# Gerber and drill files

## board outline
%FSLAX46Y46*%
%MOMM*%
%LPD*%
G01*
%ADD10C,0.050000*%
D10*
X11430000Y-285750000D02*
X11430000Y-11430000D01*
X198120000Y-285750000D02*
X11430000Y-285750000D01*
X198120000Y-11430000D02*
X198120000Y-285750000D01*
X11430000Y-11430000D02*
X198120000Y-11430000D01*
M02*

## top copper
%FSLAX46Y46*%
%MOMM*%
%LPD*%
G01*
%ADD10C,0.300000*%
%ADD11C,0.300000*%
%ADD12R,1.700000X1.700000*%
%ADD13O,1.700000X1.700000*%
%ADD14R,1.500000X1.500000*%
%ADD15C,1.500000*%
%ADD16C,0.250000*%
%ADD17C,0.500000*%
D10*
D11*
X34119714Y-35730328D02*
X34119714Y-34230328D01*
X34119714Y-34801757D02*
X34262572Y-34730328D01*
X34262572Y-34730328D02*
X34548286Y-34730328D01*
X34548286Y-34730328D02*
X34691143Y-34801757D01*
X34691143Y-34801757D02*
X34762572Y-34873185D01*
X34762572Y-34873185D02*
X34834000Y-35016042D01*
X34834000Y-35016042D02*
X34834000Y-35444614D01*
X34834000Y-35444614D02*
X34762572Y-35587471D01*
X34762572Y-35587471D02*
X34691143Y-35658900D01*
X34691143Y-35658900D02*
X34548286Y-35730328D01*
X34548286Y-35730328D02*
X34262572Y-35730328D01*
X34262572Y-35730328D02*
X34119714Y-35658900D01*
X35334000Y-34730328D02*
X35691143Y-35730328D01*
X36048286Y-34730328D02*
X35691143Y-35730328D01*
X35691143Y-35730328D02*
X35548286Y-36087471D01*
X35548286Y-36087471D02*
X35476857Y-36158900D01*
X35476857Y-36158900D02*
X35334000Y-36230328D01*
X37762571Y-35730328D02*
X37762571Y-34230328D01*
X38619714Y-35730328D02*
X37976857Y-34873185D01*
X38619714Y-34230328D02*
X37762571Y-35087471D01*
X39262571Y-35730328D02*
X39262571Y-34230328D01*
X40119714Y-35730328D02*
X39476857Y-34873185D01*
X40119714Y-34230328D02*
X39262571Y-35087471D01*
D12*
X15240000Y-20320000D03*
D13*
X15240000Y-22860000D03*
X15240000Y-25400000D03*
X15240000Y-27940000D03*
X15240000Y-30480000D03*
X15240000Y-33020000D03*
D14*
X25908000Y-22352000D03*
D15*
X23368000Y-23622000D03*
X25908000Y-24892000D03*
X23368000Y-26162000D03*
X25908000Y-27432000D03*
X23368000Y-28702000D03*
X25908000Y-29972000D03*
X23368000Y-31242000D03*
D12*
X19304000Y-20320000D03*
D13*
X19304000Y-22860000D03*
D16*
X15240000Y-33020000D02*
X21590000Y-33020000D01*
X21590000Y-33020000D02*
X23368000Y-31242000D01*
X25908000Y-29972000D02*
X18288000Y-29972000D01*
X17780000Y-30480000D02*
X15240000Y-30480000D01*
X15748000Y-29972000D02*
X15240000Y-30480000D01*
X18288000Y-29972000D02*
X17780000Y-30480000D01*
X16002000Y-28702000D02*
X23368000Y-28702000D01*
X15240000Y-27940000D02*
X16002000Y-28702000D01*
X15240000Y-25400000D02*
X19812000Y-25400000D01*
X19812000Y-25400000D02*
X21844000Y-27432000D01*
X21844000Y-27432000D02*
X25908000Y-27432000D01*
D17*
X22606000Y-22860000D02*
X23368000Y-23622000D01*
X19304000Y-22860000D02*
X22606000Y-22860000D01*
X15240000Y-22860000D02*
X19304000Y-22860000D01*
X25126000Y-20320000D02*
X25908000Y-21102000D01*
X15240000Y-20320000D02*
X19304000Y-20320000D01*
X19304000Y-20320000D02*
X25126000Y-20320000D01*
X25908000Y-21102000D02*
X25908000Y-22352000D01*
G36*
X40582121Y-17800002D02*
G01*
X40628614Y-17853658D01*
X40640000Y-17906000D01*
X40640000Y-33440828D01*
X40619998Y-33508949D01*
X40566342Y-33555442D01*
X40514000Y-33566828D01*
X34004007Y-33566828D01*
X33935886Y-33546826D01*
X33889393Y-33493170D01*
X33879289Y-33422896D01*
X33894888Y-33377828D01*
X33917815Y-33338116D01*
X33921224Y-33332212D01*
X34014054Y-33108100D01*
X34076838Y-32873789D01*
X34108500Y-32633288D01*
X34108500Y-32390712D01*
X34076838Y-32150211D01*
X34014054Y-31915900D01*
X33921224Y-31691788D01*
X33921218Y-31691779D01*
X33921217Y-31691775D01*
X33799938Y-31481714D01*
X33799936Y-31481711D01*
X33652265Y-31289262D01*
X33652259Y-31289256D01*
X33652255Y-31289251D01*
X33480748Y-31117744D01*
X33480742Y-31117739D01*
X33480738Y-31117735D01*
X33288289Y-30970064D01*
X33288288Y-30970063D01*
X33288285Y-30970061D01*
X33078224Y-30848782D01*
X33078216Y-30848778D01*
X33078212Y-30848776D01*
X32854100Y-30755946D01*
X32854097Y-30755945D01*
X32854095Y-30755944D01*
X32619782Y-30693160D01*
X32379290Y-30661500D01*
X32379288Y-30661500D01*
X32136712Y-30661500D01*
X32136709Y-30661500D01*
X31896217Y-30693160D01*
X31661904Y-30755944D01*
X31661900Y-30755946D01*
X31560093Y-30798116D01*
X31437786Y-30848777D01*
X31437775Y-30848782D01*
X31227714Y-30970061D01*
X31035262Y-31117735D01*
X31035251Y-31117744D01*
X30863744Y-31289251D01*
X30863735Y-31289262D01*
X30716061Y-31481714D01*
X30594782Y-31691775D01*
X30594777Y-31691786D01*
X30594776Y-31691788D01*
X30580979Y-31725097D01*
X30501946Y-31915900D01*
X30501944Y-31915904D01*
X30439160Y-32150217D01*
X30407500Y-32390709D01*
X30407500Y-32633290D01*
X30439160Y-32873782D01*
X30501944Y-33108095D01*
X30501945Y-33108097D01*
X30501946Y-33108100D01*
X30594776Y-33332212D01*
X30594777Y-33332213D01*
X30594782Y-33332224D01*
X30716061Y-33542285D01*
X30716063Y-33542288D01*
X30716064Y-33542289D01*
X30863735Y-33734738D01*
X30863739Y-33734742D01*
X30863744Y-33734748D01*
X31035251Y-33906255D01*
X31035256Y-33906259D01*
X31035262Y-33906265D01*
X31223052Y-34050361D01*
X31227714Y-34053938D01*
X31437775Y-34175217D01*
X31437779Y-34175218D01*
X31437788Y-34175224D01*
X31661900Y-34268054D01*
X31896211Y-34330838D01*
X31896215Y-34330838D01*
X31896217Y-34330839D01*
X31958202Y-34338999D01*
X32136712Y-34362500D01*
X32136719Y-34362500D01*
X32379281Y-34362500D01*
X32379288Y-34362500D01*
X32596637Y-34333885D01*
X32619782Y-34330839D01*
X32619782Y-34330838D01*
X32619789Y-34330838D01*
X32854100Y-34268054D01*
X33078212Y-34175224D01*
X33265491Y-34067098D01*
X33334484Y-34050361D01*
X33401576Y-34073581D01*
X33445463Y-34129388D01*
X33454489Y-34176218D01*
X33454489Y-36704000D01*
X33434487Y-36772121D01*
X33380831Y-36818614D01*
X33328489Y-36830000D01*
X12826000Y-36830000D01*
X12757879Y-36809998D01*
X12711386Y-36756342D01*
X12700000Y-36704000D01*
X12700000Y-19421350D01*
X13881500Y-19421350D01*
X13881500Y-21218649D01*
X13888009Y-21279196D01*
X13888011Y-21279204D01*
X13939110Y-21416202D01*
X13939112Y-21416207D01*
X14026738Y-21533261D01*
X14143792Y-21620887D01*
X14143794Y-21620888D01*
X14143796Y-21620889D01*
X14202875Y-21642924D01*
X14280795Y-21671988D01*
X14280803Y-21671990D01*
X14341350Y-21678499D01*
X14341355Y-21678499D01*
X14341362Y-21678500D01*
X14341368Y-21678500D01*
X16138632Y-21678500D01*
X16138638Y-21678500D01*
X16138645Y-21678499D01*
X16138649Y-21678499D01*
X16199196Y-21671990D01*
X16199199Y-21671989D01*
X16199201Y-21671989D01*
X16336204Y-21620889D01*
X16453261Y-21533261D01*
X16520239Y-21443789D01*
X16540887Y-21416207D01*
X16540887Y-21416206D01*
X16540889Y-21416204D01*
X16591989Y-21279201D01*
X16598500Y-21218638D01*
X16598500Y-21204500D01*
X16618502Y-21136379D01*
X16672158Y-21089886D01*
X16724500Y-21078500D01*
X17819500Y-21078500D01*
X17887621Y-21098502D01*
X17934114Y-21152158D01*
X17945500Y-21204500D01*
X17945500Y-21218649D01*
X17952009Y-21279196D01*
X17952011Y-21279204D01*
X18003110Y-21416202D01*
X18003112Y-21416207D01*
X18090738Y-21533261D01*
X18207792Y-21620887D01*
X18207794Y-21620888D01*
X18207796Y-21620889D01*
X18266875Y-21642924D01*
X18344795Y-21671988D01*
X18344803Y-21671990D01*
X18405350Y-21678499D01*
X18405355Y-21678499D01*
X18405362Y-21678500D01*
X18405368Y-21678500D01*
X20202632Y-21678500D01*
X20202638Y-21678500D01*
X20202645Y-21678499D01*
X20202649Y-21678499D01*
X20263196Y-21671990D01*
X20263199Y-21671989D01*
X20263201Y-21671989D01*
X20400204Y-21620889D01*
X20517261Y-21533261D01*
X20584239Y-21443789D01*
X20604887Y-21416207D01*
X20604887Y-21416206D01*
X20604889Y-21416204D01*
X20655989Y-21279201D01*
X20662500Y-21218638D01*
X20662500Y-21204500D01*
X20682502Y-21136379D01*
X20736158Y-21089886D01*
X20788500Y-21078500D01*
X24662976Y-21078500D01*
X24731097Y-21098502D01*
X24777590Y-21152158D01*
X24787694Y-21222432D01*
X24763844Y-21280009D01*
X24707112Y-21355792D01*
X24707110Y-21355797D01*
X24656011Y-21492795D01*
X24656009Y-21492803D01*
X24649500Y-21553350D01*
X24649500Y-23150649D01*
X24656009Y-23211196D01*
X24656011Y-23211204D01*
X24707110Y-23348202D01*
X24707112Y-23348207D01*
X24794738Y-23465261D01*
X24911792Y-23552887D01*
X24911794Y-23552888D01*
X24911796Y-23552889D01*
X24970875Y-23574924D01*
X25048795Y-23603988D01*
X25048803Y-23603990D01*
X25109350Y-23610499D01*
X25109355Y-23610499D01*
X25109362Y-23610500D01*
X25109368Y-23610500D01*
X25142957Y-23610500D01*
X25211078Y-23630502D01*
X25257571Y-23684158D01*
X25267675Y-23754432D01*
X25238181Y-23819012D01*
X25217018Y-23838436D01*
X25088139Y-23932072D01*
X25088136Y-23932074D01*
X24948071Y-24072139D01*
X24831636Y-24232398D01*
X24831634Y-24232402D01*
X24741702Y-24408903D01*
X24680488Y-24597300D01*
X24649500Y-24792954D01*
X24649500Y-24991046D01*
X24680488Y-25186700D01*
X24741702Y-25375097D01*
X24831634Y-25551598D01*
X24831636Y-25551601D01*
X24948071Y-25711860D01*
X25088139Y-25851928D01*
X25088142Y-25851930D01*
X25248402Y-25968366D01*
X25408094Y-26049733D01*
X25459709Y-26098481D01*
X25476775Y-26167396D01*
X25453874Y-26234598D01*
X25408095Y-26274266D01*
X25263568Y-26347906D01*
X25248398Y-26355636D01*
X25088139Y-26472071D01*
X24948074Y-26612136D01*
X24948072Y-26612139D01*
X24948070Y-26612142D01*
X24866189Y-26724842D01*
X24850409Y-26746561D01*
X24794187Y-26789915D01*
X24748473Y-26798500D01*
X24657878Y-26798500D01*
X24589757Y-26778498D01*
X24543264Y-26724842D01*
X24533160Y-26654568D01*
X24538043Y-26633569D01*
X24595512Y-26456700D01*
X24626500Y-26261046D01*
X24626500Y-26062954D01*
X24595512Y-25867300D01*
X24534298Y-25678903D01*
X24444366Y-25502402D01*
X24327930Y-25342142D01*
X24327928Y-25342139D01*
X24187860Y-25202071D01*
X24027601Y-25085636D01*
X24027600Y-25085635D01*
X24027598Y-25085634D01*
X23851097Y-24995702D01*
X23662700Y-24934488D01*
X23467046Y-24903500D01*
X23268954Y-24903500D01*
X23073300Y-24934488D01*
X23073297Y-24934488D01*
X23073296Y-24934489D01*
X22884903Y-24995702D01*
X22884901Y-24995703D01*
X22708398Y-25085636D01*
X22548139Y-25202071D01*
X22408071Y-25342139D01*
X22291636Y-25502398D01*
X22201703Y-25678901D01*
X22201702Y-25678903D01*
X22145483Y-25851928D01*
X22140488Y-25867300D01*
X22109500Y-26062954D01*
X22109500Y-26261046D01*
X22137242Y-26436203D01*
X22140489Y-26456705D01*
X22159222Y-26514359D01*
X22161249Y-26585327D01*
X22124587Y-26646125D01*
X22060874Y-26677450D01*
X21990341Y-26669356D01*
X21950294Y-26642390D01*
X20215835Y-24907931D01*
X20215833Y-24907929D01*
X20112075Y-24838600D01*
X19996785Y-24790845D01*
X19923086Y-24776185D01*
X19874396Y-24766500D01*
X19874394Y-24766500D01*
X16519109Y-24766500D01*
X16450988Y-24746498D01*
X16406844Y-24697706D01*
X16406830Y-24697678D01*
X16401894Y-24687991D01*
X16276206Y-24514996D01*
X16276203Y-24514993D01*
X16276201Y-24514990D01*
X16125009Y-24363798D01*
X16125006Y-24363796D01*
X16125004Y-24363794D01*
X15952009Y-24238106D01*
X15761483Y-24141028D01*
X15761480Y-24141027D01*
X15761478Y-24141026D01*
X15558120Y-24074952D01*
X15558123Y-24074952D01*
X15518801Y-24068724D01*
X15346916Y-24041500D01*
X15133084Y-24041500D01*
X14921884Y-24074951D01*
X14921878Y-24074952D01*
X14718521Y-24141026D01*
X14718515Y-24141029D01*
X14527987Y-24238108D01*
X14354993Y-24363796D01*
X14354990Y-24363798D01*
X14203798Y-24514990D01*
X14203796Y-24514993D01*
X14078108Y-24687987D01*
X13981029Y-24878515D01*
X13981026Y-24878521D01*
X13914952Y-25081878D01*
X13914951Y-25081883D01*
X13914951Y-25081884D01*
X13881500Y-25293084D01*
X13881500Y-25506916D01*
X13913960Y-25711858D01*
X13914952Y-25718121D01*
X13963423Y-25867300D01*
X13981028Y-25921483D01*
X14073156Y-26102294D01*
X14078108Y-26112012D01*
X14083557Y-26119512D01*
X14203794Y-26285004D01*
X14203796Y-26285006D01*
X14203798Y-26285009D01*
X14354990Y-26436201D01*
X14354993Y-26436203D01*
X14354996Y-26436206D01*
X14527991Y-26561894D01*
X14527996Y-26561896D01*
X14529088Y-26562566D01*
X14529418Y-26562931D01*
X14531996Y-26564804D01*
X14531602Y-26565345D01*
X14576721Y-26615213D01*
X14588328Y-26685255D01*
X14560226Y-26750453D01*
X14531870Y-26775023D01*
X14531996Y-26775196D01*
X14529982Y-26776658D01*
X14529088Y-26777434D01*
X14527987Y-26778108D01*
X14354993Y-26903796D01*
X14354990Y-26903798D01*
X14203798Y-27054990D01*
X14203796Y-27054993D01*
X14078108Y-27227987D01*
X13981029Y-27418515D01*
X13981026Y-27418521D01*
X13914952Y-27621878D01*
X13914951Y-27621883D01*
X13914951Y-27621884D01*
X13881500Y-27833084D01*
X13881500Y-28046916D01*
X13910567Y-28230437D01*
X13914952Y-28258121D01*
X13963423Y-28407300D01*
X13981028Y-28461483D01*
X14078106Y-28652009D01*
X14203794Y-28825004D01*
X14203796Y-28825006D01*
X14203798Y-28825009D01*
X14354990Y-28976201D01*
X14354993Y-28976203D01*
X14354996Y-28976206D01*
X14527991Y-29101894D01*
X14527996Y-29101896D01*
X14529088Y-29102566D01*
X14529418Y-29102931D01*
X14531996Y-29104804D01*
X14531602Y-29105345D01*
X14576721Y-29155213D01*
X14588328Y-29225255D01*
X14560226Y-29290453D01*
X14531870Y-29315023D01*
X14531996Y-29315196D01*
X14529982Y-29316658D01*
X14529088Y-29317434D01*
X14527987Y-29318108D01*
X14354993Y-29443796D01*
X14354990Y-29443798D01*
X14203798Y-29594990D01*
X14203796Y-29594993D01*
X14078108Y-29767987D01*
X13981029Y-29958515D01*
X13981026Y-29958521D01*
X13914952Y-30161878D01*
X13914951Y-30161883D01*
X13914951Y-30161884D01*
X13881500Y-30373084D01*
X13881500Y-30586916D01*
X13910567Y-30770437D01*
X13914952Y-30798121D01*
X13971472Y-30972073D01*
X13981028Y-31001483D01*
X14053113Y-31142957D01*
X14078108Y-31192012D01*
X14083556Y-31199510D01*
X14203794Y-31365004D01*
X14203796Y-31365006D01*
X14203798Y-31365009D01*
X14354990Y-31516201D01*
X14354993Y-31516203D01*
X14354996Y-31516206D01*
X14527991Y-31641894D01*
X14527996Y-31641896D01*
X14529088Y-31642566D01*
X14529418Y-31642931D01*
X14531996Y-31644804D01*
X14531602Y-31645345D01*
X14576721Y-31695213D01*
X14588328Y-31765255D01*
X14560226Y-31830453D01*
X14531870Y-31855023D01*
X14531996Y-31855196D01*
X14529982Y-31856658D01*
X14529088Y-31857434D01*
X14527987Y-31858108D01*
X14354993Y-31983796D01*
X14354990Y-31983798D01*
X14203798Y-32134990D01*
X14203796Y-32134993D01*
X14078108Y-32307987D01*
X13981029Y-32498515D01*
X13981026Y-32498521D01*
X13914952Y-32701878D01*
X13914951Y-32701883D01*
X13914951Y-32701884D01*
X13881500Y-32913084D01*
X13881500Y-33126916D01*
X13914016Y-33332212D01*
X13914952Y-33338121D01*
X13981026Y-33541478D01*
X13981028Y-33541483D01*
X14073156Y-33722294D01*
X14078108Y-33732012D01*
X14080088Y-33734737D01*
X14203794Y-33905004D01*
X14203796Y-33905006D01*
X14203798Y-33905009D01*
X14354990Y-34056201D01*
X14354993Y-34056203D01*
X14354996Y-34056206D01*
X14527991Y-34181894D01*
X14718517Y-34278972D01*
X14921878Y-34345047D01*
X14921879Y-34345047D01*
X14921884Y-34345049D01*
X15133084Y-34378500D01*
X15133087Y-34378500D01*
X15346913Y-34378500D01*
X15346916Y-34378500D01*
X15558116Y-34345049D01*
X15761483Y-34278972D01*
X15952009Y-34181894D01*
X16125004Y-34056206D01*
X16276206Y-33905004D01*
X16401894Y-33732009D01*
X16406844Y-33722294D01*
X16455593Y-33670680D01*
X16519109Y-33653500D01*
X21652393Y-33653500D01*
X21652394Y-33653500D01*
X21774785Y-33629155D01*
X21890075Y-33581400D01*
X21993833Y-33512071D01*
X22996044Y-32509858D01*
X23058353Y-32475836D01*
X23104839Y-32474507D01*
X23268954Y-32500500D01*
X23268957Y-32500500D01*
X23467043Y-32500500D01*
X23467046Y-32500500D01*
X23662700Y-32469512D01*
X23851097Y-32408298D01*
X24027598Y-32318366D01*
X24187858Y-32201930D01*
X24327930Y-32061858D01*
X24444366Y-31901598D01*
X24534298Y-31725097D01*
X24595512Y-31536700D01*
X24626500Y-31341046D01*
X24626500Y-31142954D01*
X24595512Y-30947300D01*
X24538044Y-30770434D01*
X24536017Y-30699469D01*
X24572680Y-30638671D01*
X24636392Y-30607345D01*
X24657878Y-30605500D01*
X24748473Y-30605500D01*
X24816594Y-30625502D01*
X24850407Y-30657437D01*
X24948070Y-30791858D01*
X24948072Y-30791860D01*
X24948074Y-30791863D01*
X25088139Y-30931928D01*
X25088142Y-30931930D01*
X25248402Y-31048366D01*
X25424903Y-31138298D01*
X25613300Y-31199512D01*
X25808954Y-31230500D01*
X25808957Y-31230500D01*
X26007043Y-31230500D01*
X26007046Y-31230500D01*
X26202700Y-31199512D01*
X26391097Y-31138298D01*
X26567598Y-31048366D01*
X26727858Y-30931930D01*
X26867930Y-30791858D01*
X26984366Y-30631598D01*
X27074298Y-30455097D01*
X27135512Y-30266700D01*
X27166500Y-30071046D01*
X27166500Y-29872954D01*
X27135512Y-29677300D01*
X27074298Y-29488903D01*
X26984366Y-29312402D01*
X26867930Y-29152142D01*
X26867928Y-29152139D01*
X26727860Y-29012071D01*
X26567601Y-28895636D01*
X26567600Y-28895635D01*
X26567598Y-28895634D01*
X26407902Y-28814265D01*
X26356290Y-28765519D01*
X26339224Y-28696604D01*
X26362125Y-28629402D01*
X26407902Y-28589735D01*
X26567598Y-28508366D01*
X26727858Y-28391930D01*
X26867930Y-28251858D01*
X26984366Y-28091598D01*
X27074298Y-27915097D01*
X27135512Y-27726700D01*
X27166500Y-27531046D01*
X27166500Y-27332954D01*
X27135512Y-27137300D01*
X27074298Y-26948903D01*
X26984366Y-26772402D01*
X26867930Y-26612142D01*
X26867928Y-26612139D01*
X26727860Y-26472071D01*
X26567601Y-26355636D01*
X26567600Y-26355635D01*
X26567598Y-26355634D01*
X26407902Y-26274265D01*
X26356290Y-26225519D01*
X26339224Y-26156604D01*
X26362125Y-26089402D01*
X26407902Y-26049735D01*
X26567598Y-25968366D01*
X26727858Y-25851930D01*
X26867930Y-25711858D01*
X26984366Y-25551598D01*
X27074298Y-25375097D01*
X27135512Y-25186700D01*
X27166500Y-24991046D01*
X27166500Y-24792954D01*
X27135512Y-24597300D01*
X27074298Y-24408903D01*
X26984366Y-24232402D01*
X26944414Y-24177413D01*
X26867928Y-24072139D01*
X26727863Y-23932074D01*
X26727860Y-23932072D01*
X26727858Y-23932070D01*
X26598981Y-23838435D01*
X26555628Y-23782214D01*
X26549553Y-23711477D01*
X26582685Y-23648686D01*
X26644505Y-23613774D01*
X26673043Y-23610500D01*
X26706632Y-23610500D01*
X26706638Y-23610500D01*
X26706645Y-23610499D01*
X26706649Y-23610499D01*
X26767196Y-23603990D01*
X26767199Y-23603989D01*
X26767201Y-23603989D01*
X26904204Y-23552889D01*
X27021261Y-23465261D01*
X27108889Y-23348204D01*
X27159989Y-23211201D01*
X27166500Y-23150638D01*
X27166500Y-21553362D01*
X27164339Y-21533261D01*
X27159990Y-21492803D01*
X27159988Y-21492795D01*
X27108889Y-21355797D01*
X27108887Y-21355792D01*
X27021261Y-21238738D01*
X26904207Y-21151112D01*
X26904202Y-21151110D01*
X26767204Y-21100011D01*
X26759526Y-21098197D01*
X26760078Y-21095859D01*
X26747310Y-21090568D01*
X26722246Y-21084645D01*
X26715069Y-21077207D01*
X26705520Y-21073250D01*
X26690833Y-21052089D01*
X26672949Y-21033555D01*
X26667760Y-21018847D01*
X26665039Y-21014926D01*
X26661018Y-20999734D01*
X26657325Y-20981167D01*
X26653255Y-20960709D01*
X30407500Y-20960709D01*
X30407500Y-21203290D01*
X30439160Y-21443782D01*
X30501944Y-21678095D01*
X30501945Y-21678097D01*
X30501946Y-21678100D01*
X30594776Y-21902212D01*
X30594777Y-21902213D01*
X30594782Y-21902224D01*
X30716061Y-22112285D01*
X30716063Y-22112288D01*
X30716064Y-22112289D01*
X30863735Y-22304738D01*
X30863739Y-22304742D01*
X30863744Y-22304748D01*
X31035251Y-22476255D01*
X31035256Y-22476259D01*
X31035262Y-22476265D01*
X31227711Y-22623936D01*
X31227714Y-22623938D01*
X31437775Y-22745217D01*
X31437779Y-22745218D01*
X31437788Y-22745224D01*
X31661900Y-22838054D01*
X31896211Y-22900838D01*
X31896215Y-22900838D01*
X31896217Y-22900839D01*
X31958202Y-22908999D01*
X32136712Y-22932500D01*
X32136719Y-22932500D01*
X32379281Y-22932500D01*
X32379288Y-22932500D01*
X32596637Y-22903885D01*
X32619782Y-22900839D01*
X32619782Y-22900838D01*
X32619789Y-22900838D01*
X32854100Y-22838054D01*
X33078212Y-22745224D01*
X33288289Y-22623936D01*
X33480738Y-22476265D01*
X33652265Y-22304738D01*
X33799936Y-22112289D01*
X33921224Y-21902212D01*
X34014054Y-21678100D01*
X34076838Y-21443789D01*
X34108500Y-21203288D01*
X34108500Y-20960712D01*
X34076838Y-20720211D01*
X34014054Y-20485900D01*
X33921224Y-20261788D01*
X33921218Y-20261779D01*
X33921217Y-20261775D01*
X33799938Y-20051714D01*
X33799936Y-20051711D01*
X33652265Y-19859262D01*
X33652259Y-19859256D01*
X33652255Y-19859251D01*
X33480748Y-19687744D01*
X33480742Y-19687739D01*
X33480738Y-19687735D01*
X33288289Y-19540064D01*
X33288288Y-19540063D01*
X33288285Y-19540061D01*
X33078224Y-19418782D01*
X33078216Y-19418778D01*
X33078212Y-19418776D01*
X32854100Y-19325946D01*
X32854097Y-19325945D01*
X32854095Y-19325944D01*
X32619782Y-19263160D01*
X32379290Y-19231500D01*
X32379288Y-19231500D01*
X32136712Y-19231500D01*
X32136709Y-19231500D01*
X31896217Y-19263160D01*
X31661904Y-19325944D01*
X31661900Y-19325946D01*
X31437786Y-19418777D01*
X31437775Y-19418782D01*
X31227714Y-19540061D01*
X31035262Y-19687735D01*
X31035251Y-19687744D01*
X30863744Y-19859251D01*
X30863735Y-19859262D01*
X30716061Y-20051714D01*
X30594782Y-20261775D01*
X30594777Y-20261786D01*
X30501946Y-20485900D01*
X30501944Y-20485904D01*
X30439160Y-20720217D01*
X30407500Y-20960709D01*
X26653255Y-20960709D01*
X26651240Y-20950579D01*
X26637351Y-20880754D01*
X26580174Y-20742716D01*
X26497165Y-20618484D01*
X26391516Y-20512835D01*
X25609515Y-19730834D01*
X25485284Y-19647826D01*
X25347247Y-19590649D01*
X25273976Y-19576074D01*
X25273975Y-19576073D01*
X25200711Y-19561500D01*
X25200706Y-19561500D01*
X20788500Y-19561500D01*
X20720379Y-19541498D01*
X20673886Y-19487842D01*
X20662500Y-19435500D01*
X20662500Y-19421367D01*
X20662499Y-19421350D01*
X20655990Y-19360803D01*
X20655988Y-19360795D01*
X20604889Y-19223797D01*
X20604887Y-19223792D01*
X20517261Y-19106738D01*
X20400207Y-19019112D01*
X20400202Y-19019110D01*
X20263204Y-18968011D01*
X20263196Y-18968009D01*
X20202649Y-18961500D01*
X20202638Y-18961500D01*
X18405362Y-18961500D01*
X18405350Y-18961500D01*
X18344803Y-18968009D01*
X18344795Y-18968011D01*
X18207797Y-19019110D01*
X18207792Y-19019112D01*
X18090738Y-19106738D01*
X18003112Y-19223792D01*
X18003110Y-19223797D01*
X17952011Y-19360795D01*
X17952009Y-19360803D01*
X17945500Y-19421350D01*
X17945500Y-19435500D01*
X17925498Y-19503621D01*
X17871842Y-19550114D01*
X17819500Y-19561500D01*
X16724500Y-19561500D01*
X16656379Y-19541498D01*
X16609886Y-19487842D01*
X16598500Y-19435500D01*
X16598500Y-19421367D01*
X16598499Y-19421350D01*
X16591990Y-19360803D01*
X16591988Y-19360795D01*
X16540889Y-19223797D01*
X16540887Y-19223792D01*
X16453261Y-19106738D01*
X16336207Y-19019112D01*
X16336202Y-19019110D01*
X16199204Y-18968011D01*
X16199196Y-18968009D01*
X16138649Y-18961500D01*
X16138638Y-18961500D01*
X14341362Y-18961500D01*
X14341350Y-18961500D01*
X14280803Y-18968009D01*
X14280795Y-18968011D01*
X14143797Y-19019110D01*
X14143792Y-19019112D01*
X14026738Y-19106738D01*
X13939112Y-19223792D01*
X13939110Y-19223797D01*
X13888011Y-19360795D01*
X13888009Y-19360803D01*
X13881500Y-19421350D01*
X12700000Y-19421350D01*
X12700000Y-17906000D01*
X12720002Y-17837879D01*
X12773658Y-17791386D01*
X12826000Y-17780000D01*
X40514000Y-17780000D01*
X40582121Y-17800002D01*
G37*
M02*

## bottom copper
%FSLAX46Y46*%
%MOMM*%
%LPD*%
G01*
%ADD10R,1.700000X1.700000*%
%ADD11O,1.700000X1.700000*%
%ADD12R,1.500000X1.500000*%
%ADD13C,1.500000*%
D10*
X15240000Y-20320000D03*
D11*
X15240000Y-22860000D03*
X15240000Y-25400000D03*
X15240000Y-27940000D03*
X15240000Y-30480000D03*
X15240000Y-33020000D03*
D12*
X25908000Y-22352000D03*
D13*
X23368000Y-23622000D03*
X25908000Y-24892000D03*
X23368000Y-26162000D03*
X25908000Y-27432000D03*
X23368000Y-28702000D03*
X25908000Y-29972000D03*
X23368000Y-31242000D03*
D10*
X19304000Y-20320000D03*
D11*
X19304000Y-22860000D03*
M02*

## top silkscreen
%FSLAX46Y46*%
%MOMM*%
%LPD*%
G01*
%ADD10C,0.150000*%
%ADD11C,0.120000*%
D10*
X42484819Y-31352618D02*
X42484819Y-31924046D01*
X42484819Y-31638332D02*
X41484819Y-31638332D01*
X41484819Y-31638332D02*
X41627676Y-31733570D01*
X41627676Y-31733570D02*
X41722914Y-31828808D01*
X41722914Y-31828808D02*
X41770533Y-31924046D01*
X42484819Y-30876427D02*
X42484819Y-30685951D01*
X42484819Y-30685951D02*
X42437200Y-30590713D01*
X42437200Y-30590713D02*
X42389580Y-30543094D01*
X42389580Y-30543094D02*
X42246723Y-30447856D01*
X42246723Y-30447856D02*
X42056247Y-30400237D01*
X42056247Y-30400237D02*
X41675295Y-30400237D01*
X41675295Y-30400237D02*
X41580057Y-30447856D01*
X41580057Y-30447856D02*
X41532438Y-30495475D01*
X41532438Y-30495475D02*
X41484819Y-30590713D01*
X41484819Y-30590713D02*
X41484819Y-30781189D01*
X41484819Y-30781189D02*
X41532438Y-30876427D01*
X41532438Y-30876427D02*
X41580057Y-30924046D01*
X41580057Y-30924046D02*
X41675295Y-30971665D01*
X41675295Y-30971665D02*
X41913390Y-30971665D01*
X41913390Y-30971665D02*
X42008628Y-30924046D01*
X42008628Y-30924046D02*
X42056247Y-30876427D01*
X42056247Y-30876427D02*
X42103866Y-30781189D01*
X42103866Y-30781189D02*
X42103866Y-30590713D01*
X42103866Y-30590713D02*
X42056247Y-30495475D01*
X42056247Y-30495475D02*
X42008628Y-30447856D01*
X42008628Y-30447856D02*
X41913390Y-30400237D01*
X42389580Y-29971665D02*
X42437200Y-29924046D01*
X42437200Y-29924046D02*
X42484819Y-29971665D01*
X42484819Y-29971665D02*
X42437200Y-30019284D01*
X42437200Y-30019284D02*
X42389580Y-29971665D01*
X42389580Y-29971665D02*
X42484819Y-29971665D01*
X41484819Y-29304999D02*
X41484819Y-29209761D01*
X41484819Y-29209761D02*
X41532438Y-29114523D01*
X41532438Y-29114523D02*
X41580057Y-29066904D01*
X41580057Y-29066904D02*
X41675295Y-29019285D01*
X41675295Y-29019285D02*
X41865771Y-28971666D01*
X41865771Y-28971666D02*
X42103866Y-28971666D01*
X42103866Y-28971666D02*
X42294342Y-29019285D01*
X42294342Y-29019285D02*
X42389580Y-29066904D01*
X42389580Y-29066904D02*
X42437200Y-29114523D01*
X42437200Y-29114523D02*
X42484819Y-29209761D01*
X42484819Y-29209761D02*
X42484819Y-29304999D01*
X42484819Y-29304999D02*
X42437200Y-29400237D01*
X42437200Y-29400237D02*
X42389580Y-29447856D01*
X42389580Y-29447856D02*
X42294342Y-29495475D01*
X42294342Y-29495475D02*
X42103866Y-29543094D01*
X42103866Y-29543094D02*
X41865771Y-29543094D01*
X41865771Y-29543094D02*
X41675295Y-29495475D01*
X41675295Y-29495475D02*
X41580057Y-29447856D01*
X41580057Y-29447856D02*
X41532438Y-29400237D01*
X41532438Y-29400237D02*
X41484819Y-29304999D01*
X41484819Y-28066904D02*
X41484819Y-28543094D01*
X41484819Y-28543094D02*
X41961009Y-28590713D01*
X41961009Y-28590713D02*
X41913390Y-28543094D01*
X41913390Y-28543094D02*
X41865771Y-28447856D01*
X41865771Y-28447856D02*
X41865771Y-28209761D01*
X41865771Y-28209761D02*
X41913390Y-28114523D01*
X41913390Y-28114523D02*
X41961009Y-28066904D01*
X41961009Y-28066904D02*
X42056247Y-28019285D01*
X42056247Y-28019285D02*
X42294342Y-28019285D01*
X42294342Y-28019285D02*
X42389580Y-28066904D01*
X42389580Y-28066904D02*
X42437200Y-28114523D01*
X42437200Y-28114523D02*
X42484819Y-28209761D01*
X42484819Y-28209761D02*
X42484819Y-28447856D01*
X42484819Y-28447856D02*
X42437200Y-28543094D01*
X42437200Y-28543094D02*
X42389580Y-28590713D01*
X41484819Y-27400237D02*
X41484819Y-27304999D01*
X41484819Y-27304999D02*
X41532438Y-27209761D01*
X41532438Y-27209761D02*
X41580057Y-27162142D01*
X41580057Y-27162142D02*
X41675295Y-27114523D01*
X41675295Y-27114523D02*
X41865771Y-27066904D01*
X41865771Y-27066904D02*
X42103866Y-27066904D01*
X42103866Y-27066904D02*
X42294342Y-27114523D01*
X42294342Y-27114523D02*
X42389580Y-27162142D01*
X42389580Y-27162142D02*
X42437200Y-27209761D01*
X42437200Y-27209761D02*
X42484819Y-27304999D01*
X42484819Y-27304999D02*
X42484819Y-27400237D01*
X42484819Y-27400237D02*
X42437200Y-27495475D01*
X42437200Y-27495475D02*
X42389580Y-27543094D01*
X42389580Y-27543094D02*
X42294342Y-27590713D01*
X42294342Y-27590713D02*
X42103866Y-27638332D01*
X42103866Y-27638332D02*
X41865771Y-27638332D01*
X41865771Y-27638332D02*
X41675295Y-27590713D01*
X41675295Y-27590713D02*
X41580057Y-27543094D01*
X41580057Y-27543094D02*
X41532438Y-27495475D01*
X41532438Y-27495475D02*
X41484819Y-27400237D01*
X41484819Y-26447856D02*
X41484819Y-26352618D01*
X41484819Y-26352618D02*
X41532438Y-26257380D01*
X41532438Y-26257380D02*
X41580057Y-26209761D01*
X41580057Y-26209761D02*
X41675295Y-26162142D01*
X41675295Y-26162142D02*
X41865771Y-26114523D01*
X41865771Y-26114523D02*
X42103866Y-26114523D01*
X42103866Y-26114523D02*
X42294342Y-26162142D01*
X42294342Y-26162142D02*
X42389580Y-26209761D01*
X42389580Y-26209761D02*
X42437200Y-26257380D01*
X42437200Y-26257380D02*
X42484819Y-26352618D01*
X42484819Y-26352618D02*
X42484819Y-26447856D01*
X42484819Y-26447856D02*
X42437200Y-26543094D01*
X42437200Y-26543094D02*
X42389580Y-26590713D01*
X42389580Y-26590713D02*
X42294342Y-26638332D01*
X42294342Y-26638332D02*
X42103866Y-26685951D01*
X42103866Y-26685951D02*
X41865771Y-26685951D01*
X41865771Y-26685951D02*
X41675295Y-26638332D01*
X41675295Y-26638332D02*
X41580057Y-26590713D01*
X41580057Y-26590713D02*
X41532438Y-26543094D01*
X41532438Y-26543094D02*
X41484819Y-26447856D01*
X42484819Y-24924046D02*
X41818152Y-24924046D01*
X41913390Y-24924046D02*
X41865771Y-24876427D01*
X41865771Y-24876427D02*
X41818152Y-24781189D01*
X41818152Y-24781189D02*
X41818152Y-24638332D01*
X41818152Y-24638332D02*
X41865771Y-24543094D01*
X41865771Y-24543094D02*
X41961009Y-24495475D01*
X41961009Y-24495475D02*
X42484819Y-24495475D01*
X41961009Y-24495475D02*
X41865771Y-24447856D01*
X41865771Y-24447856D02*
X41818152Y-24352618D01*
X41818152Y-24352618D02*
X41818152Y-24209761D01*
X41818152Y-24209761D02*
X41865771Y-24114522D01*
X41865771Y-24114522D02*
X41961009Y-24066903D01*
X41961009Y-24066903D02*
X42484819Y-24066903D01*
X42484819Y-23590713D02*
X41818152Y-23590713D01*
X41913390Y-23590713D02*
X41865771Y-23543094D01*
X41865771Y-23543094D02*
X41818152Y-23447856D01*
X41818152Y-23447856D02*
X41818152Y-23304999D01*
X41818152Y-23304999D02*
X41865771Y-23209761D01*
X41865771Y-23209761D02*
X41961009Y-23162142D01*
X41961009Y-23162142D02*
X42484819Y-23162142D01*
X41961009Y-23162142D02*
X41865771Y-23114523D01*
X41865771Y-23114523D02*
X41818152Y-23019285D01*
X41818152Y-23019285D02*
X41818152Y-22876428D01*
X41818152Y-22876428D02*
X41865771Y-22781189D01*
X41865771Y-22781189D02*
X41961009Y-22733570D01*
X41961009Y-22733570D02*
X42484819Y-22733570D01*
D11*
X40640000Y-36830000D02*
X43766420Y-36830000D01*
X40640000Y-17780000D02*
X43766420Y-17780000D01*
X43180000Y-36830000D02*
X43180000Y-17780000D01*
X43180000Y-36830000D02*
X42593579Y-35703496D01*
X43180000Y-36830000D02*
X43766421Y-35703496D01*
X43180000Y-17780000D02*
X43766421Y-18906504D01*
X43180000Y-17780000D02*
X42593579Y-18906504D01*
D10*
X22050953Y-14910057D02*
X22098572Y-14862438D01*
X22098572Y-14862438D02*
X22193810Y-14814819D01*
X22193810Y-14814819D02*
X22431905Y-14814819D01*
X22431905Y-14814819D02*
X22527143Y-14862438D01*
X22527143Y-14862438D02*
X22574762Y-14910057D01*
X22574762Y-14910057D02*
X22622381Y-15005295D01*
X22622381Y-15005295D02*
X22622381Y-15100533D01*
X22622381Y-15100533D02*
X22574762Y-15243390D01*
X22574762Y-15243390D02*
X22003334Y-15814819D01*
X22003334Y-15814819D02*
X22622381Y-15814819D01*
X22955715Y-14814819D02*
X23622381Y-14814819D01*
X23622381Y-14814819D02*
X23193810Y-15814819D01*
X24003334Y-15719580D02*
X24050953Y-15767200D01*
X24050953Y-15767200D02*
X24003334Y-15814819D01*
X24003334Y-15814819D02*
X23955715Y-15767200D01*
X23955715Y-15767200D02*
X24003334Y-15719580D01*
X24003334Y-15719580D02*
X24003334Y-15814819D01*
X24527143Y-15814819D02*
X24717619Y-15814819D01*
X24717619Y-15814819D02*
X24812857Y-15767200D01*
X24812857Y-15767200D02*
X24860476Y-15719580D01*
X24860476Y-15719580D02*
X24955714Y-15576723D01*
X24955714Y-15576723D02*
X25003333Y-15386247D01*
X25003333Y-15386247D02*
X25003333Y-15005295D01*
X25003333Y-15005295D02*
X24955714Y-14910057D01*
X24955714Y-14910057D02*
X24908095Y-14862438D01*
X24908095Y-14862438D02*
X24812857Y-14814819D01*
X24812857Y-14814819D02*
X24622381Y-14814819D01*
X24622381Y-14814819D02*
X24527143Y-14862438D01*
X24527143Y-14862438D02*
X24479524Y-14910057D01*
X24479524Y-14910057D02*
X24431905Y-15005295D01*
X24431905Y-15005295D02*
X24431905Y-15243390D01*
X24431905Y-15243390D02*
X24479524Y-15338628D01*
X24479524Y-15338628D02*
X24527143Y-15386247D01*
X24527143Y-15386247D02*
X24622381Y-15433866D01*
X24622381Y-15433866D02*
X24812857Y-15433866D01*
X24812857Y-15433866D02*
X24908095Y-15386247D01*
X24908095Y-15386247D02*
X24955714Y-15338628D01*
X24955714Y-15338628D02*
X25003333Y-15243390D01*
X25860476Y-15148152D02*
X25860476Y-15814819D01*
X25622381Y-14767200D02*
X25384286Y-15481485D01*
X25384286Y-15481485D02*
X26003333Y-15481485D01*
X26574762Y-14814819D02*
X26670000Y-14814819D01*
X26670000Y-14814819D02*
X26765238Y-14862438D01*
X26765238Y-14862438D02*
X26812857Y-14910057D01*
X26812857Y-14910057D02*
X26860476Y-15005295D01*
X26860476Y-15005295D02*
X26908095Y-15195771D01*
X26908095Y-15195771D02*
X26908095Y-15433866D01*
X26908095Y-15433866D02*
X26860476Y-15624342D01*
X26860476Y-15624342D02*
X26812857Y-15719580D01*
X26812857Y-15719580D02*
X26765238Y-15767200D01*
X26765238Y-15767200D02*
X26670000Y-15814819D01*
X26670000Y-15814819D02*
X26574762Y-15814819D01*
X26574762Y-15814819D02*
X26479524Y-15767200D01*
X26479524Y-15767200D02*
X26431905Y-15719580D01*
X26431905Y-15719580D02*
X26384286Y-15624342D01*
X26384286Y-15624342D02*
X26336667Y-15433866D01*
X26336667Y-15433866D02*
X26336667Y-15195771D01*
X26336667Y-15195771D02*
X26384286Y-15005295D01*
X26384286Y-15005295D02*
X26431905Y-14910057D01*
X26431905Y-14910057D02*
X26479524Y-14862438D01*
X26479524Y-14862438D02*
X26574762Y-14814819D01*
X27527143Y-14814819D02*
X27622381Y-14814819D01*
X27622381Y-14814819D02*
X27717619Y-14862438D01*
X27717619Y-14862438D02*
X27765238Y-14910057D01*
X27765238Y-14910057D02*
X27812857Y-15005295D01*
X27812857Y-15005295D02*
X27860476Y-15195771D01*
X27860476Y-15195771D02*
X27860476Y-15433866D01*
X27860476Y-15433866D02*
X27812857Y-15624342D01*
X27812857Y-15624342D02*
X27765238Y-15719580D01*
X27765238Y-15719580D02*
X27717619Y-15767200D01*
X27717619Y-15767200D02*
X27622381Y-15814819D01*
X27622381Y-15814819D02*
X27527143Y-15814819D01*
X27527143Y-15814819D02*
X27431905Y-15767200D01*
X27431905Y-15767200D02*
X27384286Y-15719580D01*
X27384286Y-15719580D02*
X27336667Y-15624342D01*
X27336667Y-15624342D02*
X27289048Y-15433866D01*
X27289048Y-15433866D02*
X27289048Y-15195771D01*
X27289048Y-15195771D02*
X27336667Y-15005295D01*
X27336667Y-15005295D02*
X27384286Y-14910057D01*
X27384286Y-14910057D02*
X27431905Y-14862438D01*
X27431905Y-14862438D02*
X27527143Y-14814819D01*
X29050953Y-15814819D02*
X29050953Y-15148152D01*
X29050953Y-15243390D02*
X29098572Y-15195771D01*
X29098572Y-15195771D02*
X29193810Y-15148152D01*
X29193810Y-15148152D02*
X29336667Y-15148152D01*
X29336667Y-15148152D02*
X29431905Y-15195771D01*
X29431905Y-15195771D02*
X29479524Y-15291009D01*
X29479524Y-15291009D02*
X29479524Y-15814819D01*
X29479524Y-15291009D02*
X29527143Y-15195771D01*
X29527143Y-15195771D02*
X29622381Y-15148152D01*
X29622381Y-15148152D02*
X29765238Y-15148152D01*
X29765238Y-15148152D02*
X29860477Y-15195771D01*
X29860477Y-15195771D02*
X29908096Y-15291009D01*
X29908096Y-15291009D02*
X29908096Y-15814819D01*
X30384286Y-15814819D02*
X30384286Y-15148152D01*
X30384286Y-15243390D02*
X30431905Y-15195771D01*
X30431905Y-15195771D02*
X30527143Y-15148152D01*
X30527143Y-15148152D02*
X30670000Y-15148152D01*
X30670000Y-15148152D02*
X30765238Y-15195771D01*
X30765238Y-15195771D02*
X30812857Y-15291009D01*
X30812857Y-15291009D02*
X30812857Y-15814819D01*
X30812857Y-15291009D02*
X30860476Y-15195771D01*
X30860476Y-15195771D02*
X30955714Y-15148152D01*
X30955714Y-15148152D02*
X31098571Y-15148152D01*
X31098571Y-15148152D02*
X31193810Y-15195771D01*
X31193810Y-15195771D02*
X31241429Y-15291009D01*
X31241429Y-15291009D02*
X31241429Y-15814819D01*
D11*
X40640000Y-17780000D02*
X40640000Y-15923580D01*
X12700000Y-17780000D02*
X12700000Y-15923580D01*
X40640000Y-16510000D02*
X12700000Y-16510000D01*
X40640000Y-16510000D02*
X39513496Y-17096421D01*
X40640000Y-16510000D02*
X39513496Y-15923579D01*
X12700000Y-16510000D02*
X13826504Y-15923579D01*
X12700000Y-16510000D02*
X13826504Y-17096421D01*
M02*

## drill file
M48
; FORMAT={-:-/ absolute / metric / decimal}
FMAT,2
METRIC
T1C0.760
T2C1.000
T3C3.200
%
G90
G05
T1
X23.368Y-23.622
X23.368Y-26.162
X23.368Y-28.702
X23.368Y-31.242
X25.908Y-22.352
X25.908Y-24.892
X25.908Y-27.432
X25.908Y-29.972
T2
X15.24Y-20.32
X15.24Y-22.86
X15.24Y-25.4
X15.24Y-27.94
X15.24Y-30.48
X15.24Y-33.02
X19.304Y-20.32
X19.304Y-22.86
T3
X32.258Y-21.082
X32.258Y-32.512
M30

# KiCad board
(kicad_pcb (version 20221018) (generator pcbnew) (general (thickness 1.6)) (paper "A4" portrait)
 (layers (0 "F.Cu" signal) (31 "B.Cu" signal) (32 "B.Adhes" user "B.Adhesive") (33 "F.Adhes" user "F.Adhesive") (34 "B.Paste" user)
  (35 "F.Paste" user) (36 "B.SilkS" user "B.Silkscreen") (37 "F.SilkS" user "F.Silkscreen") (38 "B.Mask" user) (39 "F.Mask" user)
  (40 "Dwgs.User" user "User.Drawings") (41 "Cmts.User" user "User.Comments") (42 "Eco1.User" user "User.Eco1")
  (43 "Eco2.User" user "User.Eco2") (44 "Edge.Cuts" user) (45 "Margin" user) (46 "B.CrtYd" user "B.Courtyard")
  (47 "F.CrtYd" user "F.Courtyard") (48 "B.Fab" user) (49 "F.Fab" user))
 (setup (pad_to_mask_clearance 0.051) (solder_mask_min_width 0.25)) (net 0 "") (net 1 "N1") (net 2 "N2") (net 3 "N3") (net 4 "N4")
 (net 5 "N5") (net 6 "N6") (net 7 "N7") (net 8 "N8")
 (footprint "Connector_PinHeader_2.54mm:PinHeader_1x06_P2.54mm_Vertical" (layer "B.Cu") (at 15.24 20.32 180)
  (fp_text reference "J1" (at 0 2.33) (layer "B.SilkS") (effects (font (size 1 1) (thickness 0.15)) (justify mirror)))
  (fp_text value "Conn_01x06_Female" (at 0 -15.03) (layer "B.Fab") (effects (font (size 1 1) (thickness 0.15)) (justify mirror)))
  (pad "1" thru_hole rect (at 0 0 180) (size 1.7 1.7) (drill 1) (layers "*.Cu" "*.Mask") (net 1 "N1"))
  (pad "2" thru_hole oval (at 0 -2.54 180) (size 1.7 1.7) (drill 1) (layers "*.Cu" "*.Mask") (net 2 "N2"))
  (pad "3" thru_hole oval (at 0 -5.08 180) (size 1.7 1.7) (drill 1) (layers "*.Cu" "*.Mask") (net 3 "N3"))
  (pad "4" thru_hole oval (at 0 -7.62 180) (size 1.7 1.7) (drill 1) (layers "*.Cu" "*.Mask") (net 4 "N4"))
  (pad "5" thru_hole oval (at 0 -10.16 180) (size 1.7 1.7) (drill 1) (layers "*.Cu" "*.Mask") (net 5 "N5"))
  (pad "6" thru_hole oval (at 0 -12.7 180) (size 1.7 1.7) (drill 1) (layers "*.Cu" "*.Mask") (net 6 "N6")))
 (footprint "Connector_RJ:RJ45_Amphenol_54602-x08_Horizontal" (layer "B.Cu") (at 25.908 22.352 -90)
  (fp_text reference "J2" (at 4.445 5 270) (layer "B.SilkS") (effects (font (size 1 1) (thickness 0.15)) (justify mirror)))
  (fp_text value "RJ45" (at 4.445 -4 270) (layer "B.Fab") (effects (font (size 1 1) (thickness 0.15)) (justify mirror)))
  (pad "" np_thru_hole circle (at -1.27 -6.35 270) (size 3.2 3.2) (drill 3.2) (layers "*.Cu" "*.Mask"))
  (pad "" np_thru_hole circle (at 10.16 -6.35 270) (size 3.2 3.2) (drill 3.2) (layers "*.Cu" "*.Mask"))
  (pad "1" thru_hole rect (at 0 0 270) (size 1.5 1.5) (drill 0.76) (layers "*.Cu" "*.Mask") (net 1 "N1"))
  (pad "2" thru_hole circle (at 1.27 2.54 270) (size 1.5 1.5) (drill 0.76) (layers "*.Cu" "*.Mask") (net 2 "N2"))
  (pad "3" thru_hole circle (at 2.54 0 270) (size 1.5 1.5) (drill 0.76) (layers "*.Cu" "*.Mask") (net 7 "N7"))
  (pad "4" thru_hole circle (at 3.81 2.54 270) (size 1.5 1.5) (drill 0.76) (layers "*.Cu" "*.Mask") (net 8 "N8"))
  (pad "5" thru_hole circle (at 5.08 0 270) (size 1.5 1.5) (drill 0.76) (layers "*.Cu" "*.Mask") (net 3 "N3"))
  (pad "6" thru_hole circle (at 6.35 2.54 270) (size 1.5 1.5) (drill 0.76) (layers "*.Cu" "*.Mask") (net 4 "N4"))
  (pad "7" thru_hole circle (at 7.62 0 270) (size 1.5 1.5) (drill 0.76) (layers "*.Cu" "*.Mask") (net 5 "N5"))
  (pad "8" thru_hole circle (at 8.89 2.54 270) (size 1.5 1.5) (drill 0.76) (layers "*.Cu" "*.Mask") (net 6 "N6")))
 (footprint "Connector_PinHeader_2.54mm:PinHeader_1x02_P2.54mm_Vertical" (layer "B.Cu") (at 19.304 20.32 180)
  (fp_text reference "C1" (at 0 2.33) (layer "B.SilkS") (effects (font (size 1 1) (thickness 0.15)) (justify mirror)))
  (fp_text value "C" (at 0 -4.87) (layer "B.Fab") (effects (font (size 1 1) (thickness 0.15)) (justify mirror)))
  (pad "1" thru_hole rect (at 0 0 180) (size 1.7 1.7) (drill 1) (layers "*.Cu" "*.Mask") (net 1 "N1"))
  (pad "2" thru_hole oval (at 0 -2.54 180) (size 1.7 1.7) (drill 1) (layers "*.Cu" "*.Mask") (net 2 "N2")))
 (gr_line (start 11.43 285.75) (end 11.43 11.43) (stroke (width 0.05) (type solid)) (layer "Edge.Cuts"))
 (gr_line (start 198.12 285.75) (end 11.43 285.75) (stroke (width 0.05) (type solid)) (layer "Edge.Cuts"))
 (gr_line (start 198.12 11.43) (end 198.12 285.75) (stroke (width 0.05) (type solid)) (layer "Edge.Cuts"))
 (gr_line (start 11.43 11.43) (end 198.12 11.43) (stroke (width 0.05) (type solid)) (layer "Edge.Cuts"))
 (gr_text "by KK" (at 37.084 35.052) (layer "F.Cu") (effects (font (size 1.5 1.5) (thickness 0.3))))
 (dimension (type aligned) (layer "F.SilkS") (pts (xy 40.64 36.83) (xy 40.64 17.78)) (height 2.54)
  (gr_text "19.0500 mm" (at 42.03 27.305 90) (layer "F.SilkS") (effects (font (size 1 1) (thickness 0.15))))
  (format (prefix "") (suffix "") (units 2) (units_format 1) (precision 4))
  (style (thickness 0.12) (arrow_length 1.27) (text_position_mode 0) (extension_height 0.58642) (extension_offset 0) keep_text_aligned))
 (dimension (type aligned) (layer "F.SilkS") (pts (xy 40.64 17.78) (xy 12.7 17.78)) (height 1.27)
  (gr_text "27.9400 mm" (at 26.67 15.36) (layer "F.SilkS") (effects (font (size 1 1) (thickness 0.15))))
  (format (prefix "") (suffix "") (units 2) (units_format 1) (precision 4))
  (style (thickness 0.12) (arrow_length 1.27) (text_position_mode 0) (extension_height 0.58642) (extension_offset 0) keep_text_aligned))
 (segment (start 15.24 33.02) (end 21.59 33.02) (width 0.25) (layer "F.Cu") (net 6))
 (segment (start 21.59 33.02) (end 23.368 31.242) (width 0.25) (layer "F.Cu") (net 6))
 (segment (start 25.908 29.972) (end 18.288 29.972) (width 0.25) (layer "F.Cu") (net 5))
 (segment (start 17.78 30.48) (end 15.24 30.48) (width 0.25) (layer "F.Cu") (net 5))
 (segment (start 15.748 29.972) (end 15.24 30.48) (width 0.25) (layer "F.Cu") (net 5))
 (segment (start 18.288 29.972) (end 17.78 30.48) (width 0.25) (layer "F.Cu") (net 5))
 (segment (start 16.002 28.702) (end 23.368 28.702) (width 0.25) (layer "F.Cu") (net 4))
 (segment (start 15.24 27.94) (end 16.002 28.702) (width 0.25) (layer "F.Cu") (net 4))
 (segment (start 15.24 25.4) (end 19.812 25.4) (width 0.25) (layer "F.Cu") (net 3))
 (segment (start 19.812 25.4) (end 21.844 27.432) (width 0.25) (layer "F.Cu") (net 3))
 (segment (start 21.844 27.432) (end 25.908 27.432) (width 0.25) (layer "F.Cu") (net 3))
 (segment (start 22.606 22.86) (end 23.368 23.622) (width 0.5) (layer "F.Cu") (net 2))
 (segment (start 19.304 22.86) (end 22.606 22.86) (width 0.5) (layer "F.Cu") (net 2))
 (segment (start 15.24 22.86) (end 19.304 22.86) (width 0.5) (layer "F.Cu") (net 2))
 (segment (start 25.126 20.32) (end 25.908 21.102) (width 0.5) (layer "F.Cu") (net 1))
 (segment (start 15.24 20.32) (end 19.304 20.32) (width 0.5) (layer "F.Cu") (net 1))
 (segment (start 19.304 20.32) (end 25.126 20.32) (width 0.5) (layer "F.Cu") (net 1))
 (segment (start 25.908 21.102) (end 25.908 22.352) (width 0.5) (layer "F.Cu") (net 1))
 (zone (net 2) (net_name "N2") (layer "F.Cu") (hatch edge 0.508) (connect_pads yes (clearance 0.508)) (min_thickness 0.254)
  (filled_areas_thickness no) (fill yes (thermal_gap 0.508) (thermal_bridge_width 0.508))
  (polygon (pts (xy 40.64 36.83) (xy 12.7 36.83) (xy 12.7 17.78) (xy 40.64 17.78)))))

